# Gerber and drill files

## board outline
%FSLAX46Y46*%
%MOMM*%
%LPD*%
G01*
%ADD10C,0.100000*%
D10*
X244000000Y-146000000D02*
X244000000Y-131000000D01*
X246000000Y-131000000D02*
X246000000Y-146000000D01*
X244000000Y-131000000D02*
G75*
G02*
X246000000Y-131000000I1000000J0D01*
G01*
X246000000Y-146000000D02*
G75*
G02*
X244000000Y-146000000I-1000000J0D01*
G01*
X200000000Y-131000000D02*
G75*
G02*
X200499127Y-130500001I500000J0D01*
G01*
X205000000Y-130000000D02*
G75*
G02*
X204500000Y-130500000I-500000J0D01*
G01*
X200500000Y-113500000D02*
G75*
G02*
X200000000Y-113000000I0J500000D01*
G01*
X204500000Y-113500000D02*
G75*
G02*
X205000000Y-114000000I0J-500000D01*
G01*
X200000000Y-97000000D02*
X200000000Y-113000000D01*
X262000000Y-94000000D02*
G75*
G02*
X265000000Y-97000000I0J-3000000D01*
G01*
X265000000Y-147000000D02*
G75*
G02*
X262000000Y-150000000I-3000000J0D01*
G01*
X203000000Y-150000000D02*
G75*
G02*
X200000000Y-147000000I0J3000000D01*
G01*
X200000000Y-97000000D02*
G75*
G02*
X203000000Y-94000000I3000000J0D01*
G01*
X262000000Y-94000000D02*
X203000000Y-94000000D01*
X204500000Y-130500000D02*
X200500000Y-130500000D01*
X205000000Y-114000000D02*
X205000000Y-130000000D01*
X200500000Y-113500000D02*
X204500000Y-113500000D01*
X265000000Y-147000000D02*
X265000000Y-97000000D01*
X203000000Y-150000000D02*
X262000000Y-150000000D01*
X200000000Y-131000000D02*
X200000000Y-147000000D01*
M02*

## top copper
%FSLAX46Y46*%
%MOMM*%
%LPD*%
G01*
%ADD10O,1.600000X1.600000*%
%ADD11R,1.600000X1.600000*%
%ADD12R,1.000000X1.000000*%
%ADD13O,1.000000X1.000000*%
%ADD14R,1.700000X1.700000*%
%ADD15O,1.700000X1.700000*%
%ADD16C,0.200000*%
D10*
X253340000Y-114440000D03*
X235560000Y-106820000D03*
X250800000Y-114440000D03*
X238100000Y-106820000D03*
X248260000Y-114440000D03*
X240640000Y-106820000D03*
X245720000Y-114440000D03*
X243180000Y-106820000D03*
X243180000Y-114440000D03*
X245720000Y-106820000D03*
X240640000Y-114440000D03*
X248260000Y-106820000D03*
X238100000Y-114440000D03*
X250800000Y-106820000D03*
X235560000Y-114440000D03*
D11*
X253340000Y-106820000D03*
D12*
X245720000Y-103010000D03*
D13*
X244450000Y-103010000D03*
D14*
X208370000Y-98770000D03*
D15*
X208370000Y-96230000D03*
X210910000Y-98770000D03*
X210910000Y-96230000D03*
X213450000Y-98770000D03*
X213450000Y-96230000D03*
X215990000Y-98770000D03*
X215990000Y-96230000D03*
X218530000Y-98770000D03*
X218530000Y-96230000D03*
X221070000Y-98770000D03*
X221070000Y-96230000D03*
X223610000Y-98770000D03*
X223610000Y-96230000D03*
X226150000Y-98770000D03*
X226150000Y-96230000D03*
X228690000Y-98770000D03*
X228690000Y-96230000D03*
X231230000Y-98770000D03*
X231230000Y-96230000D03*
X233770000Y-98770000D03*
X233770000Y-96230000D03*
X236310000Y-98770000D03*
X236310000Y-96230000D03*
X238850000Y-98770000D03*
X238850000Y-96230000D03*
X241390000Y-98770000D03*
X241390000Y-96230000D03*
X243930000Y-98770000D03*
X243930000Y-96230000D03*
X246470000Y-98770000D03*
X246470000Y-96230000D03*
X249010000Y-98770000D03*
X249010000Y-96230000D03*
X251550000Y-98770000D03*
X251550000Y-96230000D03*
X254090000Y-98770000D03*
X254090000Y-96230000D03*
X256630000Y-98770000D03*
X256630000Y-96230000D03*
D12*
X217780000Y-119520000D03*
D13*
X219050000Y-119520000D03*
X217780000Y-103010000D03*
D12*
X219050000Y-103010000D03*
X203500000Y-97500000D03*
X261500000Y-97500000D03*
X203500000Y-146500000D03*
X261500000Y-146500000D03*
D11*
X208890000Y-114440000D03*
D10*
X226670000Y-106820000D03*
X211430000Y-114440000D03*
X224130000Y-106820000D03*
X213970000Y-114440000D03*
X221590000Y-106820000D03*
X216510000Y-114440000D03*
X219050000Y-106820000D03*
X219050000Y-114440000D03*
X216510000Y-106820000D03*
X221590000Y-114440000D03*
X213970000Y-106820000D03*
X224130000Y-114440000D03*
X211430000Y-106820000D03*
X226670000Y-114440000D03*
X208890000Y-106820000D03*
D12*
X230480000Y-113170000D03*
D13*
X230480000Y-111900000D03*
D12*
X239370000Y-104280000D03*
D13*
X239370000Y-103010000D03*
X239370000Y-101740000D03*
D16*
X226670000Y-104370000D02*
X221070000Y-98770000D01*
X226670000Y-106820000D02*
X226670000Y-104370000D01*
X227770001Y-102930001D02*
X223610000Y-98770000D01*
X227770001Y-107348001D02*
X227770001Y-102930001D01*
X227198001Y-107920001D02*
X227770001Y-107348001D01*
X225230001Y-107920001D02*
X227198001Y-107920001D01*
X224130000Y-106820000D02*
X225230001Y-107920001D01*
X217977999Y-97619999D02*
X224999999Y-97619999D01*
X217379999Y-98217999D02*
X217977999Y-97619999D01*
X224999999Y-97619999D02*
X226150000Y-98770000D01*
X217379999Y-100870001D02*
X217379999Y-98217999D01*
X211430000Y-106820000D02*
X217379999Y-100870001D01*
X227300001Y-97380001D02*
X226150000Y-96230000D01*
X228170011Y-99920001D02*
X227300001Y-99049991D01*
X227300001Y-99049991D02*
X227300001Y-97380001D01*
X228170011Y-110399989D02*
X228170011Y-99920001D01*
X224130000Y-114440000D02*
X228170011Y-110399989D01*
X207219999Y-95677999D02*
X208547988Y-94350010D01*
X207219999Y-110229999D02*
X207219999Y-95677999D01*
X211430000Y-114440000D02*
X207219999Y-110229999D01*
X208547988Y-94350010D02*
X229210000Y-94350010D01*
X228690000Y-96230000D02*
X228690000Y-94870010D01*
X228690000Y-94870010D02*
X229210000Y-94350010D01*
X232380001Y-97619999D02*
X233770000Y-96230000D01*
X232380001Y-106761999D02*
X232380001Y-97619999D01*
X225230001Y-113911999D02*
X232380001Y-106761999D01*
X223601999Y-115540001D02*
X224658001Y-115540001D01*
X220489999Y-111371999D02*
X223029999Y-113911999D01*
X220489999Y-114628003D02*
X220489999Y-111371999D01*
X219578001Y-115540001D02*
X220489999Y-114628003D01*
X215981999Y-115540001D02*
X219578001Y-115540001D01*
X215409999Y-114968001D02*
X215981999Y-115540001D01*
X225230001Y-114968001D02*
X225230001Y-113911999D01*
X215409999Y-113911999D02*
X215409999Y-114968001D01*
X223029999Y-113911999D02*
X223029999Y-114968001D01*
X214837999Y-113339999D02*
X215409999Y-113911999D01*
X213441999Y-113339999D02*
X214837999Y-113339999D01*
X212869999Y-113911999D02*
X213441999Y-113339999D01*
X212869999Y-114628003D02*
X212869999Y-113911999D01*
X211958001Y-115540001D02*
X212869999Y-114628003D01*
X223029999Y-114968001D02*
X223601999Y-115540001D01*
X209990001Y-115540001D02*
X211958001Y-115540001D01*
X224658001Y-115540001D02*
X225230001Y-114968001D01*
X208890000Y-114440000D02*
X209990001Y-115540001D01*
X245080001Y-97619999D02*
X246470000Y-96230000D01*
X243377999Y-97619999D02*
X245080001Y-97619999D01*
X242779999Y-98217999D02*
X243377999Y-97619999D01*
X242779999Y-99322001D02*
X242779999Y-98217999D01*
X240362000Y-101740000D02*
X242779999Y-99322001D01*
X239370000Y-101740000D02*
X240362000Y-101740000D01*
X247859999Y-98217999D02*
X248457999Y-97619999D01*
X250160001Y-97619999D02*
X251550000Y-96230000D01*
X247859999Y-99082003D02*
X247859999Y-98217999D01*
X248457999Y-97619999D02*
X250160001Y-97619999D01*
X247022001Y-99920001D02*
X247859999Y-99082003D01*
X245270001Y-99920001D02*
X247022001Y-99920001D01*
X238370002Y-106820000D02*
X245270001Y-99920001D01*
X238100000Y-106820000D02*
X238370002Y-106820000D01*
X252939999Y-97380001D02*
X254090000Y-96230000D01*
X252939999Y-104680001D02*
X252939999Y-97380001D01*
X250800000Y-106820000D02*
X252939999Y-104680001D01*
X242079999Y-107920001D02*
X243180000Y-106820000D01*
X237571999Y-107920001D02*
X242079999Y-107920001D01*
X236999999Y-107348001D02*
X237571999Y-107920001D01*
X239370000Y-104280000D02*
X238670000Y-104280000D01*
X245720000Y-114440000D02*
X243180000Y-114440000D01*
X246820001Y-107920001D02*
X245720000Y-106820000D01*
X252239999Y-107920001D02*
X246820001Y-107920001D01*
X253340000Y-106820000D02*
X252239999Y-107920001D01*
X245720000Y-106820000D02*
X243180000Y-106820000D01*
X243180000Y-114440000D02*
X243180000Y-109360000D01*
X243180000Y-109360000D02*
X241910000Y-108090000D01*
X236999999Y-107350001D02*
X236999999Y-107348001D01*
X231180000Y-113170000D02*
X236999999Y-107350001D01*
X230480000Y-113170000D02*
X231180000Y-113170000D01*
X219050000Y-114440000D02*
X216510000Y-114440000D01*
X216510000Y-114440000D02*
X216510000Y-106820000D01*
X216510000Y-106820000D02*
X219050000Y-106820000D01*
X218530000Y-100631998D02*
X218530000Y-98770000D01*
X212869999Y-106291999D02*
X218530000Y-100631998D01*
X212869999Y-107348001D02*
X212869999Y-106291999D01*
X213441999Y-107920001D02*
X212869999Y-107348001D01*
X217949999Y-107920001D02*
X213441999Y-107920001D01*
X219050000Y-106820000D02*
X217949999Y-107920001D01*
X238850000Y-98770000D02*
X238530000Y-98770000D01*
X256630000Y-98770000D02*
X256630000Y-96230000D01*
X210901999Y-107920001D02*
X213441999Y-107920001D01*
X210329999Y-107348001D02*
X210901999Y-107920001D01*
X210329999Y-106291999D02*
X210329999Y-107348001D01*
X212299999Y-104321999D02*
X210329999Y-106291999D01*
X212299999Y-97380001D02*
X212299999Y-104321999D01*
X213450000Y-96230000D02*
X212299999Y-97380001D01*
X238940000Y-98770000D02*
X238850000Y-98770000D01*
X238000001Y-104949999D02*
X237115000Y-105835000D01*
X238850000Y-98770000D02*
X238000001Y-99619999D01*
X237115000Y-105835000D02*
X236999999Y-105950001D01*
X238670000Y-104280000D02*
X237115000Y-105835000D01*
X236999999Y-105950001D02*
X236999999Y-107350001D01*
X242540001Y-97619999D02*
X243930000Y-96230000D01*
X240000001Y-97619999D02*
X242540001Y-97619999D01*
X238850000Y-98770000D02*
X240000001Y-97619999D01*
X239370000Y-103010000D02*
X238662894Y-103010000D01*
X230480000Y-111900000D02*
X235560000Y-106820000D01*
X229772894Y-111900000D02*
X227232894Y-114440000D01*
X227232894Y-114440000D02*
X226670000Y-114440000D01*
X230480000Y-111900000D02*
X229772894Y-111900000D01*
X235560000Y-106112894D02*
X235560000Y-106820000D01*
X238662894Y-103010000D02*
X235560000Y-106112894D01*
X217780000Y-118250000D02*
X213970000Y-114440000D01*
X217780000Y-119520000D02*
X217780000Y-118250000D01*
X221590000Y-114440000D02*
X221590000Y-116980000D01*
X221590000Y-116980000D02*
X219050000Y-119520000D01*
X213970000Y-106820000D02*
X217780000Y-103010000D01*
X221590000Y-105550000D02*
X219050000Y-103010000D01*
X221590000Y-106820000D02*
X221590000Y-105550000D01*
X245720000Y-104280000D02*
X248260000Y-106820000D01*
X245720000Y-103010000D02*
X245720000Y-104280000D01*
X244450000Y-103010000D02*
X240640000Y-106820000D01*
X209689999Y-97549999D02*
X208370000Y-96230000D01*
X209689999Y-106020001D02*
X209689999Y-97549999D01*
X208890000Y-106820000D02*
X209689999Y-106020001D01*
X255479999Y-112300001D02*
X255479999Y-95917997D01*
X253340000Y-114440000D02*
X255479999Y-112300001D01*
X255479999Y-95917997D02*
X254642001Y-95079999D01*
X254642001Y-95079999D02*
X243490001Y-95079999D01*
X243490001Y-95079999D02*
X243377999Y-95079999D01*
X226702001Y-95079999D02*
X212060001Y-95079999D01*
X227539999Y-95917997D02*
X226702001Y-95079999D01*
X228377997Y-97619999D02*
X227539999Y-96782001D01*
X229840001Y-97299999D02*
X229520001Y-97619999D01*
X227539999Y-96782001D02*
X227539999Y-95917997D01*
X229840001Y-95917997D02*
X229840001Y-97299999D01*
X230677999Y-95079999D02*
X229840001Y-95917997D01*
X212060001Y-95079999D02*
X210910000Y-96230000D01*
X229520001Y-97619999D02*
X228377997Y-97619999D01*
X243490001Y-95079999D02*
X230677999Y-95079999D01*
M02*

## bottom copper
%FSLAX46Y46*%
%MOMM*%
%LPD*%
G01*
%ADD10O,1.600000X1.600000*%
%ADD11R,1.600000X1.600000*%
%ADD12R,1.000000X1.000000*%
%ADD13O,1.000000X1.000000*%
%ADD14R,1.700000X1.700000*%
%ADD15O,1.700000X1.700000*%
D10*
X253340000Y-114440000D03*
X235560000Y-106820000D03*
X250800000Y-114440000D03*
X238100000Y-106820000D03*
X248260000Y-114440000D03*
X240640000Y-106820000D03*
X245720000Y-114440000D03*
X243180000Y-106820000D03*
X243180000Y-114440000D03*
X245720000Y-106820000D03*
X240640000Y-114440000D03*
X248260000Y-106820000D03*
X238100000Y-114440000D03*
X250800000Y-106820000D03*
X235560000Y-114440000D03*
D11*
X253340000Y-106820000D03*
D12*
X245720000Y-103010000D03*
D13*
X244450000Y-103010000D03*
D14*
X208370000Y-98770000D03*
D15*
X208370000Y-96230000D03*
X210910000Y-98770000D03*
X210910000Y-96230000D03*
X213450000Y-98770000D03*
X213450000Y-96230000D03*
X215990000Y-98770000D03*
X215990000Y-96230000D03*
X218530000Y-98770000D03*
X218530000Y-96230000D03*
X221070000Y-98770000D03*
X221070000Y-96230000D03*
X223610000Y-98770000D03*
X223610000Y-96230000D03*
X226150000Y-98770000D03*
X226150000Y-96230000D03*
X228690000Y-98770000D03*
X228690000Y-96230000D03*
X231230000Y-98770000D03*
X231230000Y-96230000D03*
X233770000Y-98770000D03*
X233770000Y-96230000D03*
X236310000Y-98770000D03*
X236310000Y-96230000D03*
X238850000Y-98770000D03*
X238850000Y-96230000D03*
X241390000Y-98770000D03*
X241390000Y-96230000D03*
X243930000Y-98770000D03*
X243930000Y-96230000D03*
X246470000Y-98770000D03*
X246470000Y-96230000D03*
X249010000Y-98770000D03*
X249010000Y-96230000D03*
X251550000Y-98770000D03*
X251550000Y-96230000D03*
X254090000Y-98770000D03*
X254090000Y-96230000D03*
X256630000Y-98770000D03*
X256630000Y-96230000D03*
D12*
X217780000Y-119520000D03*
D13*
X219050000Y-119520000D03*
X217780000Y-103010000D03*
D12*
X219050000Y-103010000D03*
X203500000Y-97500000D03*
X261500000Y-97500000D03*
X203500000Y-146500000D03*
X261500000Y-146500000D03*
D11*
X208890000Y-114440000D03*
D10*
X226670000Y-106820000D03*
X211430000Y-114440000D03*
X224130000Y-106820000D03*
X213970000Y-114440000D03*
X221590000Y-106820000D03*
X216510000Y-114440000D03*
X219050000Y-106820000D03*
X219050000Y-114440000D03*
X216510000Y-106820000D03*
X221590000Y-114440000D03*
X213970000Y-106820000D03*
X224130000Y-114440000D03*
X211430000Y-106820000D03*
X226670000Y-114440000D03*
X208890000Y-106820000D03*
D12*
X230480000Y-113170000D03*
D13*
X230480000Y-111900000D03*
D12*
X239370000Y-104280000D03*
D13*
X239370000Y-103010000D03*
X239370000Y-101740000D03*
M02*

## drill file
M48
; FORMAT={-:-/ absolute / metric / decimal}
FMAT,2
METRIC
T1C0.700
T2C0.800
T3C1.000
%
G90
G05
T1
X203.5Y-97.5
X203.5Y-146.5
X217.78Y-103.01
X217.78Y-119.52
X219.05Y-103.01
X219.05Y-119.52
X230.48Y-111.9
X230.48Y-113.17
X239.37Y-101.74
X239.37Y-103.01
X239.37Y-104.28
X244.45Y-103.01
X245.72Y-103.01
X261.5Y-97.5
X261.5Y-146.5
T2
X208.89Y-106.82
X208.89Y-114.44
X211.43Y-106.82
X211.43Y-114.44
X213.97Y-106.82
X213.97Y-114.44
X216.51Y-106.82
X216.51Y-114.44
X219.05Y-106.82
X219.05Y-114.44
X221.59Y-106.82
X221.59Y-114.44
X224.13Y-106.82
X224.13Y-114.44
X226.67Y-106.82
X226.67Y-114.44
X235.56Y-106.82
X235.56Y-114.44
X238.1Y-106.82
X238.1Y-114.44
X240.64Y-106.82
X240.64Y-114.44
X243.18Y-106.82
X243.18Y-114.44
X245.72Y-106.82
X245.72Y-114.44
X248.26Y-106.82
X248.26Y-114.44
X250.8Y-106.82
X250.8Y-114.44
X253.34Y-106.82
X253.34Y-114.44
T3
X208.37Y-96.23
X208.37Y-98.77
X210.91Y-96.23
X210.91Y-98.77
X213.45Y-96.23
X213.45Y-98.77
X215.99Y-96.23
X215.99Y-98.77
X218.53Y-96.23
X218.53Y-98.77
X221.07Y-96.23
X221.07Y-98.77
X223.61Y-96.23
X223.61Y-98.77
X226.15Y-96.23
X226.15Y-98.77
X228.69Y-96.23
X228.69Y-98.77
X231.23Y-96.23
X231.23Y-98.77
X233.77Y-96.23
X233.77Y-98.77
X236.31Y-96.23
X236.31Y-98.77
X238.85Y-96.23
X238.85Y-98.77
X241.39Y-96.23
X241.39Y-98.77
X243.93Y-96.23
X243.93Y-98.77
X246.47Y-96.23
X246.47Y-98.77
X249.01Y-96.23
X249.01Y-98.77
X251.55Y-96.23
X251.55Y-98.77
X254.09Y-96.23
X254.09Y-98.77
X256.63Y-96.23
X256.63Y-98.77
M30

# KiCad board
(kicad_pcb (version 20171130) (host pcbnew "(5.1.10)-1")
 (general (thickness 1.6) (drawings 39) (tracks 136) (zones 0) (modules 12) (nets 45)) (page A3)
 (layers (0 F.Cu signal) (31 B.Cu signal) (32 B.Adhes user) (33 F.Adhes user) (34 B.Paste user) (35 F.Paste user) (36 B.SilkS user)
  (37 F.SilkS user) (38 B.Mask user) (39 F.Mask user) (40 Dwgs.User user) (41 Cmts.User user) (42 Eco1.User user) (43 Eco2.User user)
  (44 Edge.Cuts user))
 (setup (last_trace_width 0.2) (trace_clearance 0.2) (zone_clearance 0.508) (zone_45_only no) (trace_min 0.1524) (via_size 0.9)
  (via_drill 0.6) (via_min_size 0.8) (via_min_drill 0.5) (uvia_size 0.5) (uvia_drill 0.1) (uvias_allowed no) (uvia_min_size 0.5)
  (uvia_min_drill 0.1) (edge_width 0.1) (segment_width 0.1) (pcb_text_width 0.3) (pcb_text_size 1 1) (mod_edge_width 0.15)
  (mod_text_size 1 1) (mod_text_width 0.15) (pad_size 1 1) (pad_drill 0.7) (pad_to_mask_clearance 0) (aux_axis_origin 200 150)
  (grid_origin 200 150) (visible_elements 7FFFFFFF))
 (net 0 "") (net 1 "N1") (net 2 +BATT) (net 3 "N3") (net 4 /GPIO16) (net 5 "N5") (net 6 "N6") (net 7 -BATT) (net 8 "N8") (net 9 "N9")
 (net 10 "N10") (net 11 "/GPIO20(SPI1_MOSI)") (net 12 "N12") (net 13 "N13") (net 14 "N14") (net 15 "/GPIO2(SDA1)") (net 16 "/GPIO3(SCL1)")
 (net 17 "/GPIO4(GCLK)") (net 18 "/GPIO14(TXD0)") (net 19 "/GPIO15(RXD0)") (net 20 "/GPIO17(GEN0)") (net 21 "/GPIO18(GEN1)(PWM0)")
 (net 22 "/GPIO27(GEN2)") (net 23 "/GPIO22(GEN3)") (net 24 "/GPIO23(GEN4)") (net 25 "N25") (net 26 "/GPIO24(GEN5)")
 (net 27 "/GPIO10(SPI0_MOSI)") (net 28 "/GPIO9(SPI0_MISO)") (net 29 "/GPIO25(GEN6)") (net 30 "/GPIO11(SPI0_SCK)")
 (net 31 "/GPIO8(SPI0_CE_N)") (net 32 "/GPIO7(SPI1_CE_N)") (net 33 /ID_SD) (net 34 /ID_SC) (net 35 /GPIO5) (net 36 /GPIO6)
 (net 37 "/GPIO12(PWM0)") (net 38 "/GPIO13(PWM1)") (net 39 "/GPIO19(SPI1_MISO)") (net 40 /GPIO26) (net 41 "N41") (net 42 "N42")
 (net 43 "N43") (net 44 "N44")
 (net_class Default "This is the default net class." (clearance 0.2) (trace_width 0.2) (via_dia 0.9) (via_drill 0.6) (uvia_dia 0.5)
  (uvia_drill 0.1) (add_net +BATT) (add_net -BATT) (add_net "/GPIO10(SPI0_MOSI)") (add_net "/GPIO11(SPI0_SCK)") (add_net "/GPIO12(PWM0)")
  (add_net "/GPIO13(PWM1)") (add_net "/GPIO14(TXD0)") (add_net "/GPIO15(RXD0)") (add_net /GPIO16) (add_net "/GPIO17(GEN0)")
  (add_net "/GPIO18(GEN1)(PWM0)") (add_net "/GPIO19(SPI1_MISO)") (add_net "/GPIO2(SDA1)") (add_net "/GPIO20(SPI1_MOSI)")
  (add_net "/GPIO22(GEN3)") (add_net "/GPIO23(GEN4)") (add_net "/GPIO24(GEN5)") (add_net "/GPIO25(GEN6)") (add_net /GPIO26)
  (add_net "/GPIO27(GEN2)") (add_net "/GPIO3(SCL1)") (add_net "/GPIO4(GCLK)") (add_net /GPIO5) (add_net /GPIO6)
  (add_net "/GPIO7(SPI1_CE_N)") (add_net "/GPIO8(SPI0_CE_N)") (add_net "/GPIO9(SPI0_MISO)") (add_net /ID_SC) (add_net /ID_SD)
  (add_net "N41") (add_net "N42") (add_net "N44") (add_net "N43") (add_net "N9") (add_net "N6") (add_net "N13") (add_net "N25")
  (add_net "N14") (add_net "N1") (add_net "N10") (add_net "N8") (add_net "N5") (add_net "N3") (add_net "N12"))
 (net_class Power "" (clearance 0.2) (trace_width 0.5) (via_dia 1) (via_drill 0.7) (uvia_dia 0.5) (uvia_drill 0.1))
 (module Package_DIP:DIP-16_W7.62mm (layer F.Cu) (at 253.34 106.82 270)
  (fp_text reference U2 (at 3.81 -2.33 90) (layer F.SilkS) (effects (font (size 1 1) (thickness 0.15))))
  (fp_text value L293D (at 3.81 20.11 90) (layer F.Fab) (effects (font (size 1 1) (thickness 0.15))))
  (pad 16 thru_hole oval (at 7.62 0 270) (size 1.6 1.6) (drill 0.8) (layers *.Cu *.Mask) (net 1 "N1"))
  (pad 8 thru_hole oval (at 0 17.78 270) (size 1.6 1.6) (drill 0.8) (layers *.Cu *.Mask) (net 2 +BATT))
  (pad 15 thru_hole oval (at 7.62 2.54 270) (size 1.6 1.6) (drill 0.8) (layers *.Cu *.Mask) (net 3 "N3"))
  (pad 7 thru_hole oval (at 0 15.24 270) (size 1.6 1.6) (drill 0.8) (layers *.Cu *.Mask) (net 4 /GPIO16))
  (pad 14 thru_hole oval (at 7.62 5.08 270) (size 1.6 1.6) (drill 0.8) (layers *.Cu *.Mask) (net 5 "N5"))
  (pad 6 thru_hole oval (at 0 12.7 270) (size 1.6 1.6) (drill 0.8) (layers *.Cu *.Mask) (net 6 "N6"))
  (pad 13 thru_hole oval (at 7.62 7.62 270) (size 1.6 1.6) (drill 0.8) (layers *.Cu *.Mask) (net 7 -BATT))
  (pad 5 thru_hole oval (at 0 10.16 270) (size 1.6 1.6) (drill 0.8) (layers *.Cu *.Mask) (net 7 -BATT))
  (pad 12 thru_hole oval (at 7.62 10.16 270) (size 1.6 1.6) (drill 0.8) (layers *.Cu *.Mask) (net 7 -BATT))
  (pad 4 thru_hole oval (at 0 7.62 270) (size 1.6 1.6) (drill 0.8) (layers *.Cu *.Mask) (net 7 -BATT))
  (pad 11 thru_hole oval (at 7.62 12.7 270) (size 1.6 1.6) (drill 0.8) (layers *.Cu *.Mask) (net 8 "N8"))
  (pad 3 thru_hole oval (at 0 5.08 270) (size 1.6 1.6) (drill 0.8) (layers *.Cu *.Mask) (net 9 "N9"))
  (pad 10 thru_hole oval (at 7.62 15.24 270) (size 1.6 1.6) (drill 0.8) (layers *.Cu *.Mask) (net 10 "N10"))
  (pad 2 thru_hole oval (at 0 2.54 270) (size 1.6 1.6) (drill 0.8) (layers *.Cu *.Mask) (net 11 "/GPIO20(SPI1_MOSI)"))
  (pad 9 thru_hole oval (at 7.62 17.78 270) (size 1.6 1.6) (drill 0.8) (layers *.Cu *.Mask) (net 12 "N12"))
  (pad 1 thru_hole rect (at 0 0 270) (size 1.6 1.6) (drill 0.8) (layers *.Cu *.Mask) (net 7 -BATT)))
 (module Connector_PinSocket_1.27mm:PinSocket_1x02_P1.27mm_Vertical (layer F.Cu) (at 245.72 103.01 270)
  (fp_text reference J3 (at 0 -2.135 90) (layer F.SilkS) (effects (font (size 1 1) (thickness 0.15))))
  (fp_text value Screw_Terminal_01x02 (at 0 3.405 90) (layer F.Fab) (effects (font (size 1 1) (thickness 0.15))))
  (pad 1 thru_hole rect (at 0 0 270) (size 1 1) (drill 0.7) (layers *.Cu *.Mask) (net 9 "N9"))
  (pad 2 thru_hole oval (at 0 1.27 270) (size 1 1) (drill 0.7) (layers *.Cu *.Mask) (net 6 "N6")))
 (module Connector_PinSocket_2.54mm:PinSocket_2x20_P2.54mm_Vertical (layer B.Cu) (at 208.37 98.77 270)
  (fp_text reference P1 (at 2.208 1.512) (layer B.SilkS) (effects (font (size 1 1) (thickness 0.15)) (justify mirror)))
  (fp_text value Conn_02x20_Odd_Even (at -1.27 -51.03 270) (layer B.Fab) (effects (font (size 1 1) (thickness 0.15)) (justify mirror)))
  (pad 1 thru_hole rect (at 0 0 270) (size 1.7 1.7) (drill 1) (layers *.Cu *.Mask) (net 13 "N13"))
  (pad 2 thru_hole oval (at -2.54 0 270) (size 1.7 1.7) (drill 1) (layers *.Cu *.Mask) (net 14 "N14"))
  (pad 3 thru_hole oval (at 0 -2.54 270) (size 1.7 1.7) (drill 1) (layers *.Cu *.Mask) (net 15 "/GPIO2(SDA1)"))
  (pad 4 thru_hole oval (at -2.54 -2.54 270) (size 1.7 1.7) (drill 1) (layers *.Cu *.Mask) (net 1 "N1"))
  (pad 5 thru_hole oval (at 0 -5.08 270) (size 1.7 1.7) (drill 1) (layers *.Cu *.Mask) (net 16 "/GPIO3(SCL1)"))
  (pad 6 thru_hole oval (at -2.54 -5.08 270) (size 1.7 1.7) (drill 1) (layers *.Cu *.Mask) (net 7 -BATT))
  (pad 7 thru_hole oval (at 0 -7.62 270) (size 1.7 1.7) (drill 1) (layers *.Cu *.Mask) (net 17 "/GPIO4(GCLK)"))
  (pad 8 thru_hole oval (at -2.54 -7.62 270) (size 1.7 1.7) (drill 1) (layers *.Cu *.Mask) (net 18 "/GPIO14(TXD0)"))
  (pad 9 thru_hole oval (at 0 -10.16 270) (size 1.7 1.7) (drill 1) (layers *.Cu *.Mask) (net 7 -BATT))
  (pad 10 thru_hole oval (at -2.54 -10.16 270) (size 1.7 1.7) (drill 1) (layers *.Cu *.Mask) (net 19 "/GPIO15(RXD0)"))
  (pad 11 thru_hole oval (at 0 -12.7 270) (size 1.7 1.7) (drill 1) (layers *.Cu *.Mask) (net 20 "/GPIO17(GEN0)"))
  (pad 12 thru_hole oval (at -2.54 -12.7 270) (size 1.7 1.7) (drill 1) (layers *.Cu *.Mask) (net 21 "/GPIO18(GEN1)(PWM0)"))
  (pad 13 thru_hole oval (at 0 -15.24 270) (size 1.7 1.7) (drill 1) (layers *.Cu *.Mask) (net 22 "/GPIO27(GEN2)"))
  (pad 14 thru_hole oval (at -2.54 -15.24 270) (size 1.7 1.7) (drill 1) (layers *.Cu *.Mask) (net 7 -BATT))
  (pad 15 thru_hole oval (at 0 -17.78 270) (size 1.7 1.7) (drill 1) (layers *.Cu *.Mask) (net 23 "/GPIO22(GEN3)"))
  (pad 16 thru_hole oval (at -2.54 -17.78 270) (size 1.7 1.7) (drill 1) (layers *.Cu *.Mask) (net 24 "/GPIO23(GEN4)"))
  (pad 17 thru_hole oval (at 0 -20.32 270) (size 1.7 1.7) (drill 1) (layers *.Cu *.Mask) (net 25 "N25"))
  (pad 18 thru_hole oval (at -2.54 -20.32 270) (size 1.7 1.7) (drill 1) (layers *.Cu *.Mask) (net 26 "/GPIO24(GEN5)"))
  (pad 19 thru_hole oval (at 0 -22.86 270) (size 1.7 1.7) (drill 1) (layers *.Cu *.Mask) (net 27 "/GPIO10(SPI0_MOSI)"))
  (pad 20 thru_hole oval (at -2.54 -22.86 270) (size 1.7 1.7) (drill 1) (layers *.Cu *.Mask) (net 7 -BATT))
  (pad 21 thru_hole oval (at 0 -25.4 270) (size 1.7 1.7) (drill 1) (layers *.Cu *.Mask) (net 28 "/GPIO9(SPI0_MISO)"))
  (pad 22 thru_hole oval (at -2.54 -25.4 270) (size 1.7 1.7) (drill 1) (layers *.Cu *.Mask) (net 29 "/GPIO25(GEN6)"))
  (pad 23 thru_hole oval (at 0 -27.94 270) (size 1.7 1.7) (drill 1) (layers *.Cu *.Mask) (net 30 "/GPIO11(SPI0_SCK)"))
  (pad 24 thru_hole oval (at -2.54 -27.94 270) (size 1.7 1.7) (drill 1) (layers *.Cu *.Mask) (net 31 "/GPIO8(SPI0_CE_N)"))
  (pad 25 thru_hole oval (at 0 -30.48 270) (size 1.7 1.7) (drill 1) (layers *.Cu *.Mask) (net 7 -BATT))
  (pad 26 thru_hole oval (at -2.54 -30.48 270) (size 1.7 1.7) (drill 1) (layers *.Cu *.Mask) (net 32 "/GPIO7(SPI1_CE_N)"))
  (pad 27 thru_hole oval (at 0 -33.02 270) (size 1.7 1.7) (drill 1) (layers *.Cu *.Mask) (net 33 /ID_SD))
  (pad 28 thru_hole oval (at -2.54 -33.02 270) (size 1.7 1.7) (drill 1) (layers *.Cu *.Mask) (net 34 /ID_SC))
  (pad 29 thru_hole oval (at 0 -35.56 270) (size 1.7 1.7) (drill 1) (layers *.Cu *.Mask) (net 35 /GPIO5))
  (pad 30 thru_hole oval (at -2.54 -35.56 270) (size 1.7 1.7) (drill 1) (layers *.Cu *.Mask) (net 7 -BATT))
  (pad 31 thru_hole oval (at 0 -38.1 270) (size 1.7 1.7) (drill 1) (layers *.Cu *.Mask) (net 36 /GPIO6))
  (pad 32 thru_hole oval (at -2.54 -38.1 270) (size 1.7 1.7) (drill 1) (layers *.Cu *.Mask) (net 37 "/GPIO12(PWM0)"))
  (pad 33 thru_hole oval (at 0 -40.64 270) (size 1.7 1.7) (drill 1) (layers *.Cu *.Mask) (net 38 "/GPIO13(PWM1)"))
  (pad 34 thru_hole oval (at -2.54 -40.64 270) (size 1.7 1.7) (drill 1) (layers *.Cu *.Mask) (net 7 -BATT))
  (pad 35 thru_hole oval (at 0 -43.18 270) (size 1.7 1.7) (drill 1) (layers *.Cu *.Mask) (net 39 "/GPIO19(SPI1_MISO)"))
  (pad 36 thru_hole oval (at -2.54 -43.18 270) (size 1.7 1.7) (drill 1) (layers *.Cu *.Mask) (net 4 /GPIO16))
  (pad 37 thru_hole oval (at 0 -45.72 270) (size 1.7 1.7) (drill 1) (layers *.Cu *.Mask) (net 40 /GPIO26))
  (pad 38 thru_hole oval (at -2.54 -45.72 270) (size 1.7 1.7) (drill 1) (layers *.Cu *.Mask) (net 11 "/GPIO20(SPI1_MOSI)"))
  (pad 39 thru_hole oval (at 0 -48.26 270) (size 1.7 1.7) (drill 1) (layers *.Cu *.Mask) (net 7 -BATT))
  (pad 40 thru_hole oval (at -2.54 -48.26 270) (size 1.7 1.7) (drill 1) (layers *.Cu *.Mask) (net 7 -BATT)))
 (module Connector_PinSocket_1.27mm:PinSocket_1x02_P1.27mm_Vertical (layer F.Cu) (at 217.78 119.52 90)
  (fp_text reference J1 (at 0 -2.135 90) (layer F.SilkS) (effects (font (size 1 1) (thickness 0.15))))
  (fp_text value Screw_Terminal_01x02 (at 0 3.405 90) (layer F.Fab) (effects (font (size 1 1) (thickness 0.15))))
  (pad 1 thru_hole rect (at 0 0 90) (size 1 1) (drill 0.7) (layers *.Cu *.Mask) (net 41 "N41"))
  (pad 2 thru_hole oval (at 0 1.27 90) (size 1 1) (drill 0.7) (layers *.Cu *.Mask) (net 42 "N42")))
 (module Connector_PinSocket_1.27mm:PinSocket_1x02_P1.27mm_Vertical (layer F.Cu) (at 219.05 103.01 270)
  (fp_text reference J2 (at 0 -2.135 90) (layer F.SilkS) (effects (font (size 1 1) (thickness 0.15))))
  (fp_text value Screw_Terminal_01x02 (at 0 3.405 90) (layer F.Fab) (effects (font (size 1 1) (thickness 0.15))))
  (pad 2 thru_hole oval (at 0 1.27 270) (size 1 1) (drill 0.7) (layers *.Cu *.Mask) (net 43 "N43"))
  (pad 1 thru_hole rect (at 0 0 270) (size 1 1) (drill 0.7) (layers *.Cu *.Mask) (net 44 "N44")))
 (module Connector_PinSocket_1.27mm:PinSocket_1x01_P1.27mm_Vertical (layer F.Cu) (at 203.5 97.5 180)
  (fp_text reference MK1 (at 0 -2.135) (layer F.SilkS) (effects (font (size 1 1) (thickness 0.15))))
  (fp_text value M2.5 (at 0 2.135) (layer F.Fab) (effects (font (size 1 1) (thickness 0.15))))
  (pad 1 thru_hole rect (at 0 0 180) (size 1 1) (drill 0.7) (layers *.Cu *.Mask)))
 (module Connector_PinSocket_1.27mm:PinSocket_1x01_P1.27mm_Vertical (layer F.Cu) (at 261.5 97.5 180)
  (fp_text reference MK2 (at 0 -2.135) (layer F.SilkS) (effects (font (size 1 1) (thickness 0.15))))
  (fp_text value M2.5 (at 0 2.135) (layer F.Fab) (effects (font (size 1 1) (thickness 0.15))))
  (pad 1 thru_hole rect (at 0 0 180) (size 1 1) (drill 0.7) (layers *.Cu *.Mask)))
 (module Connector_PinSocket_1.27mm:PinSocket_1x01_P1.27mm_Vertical (layer F.Cu) (at 203.5 146.5)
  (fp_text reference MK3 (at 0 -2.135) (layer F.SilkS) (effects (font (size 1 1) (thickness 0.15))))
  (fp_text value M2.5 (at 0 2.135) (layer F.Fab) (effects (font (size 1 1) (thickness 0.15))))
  (pad 1 thru_hole rect (at 0 0) (size 1 1) (drill 0.7) (layers *.Cu *.Mask)))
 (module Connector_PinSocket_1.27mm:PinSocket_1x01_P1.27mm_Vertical (layer F.Cu) (at 261.5 146.5)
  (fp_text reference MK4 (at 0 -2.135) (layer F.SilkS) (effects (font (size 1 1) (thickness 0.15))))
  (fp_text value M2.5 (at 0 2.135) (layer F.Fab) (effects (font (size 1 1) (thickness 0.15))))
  (pad 1 thru_hole rect (at 0 0) (size 1 1) (drill 0.7) (layers *.Cu *.Mask)))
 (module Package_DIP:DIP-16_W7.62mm (layer F.Cu) (at 208.89 114.44 90)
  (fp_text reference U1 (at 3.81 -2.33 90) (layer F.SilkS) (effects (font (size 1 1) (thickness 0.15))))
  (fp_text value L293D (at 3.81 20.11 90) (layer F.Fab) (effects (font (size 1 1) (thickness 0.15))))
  (pad 1 thru_hole rect (at 0 0 90) (size 1.6 1.6) (drill 0.8) (layers *.Cu *.Mask) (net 29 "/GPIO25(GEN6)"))
  (pad 9 thru_hole oval (at 7.62 17.78 90) (size 1.6 1.6) (drill 0.8) (layers *.Cu *.Mask) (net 20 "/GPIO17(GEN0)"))
  (pad 2 thru_hole oval (at 0 2.54 90) (size 1.6 1.6) (drill 0.8) (layers *.Cu *.Mask) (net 26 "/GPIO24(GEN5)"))
  (pad 10 thru_hole oval (at 7.62 15.24 90) (size 1.6 1.6) (drill 0.8) (layers *.Cu *.Mask) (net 22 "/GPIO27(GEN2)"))
  (pad 3 thru_hole oval (at 0 5.08 90) (size 1.6 1.6) (drill 0.8) (layers *.Cu *.Mask) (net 41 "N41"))
  (pad 11 thru_hole oval (at 7.62 12.7 90) (size 1.6 1.6) (drill 0.8) (layers *.Cu *.Mask) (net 44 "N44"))
  (pad 4 thru_hole oval (at 0 7.62 90) (size 1.6 1.6) (drill 0.8) (layers *.Cu *.Mask) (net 7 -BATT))
  (pad 12 thru_hole oval (at 7.62 10.16 90) (size 1.6 1.6) (drill 0.8) (layers *.Cu *.Mask) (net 7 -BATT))
  (pad 5 thru_hole oval (at 0 10.16 90) (size 1.6 1.6) (drill 0.8) (layers *.Cu *.Mask) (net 7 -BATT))
  (pad 13 thru_hole oval (at 7.62 7.62 90) (size 1.6 1.6) (drill 0.8) (layers *.Cu *.Mask) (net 7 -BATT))
  (pad 6 thru_hole oval (at 0 12.7 90) (size 1.6 1.6) (drill 0.8) (layers *.Cu *.Mask) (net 42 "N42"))
  (pad 14 thru_hole oval (at 7.62 5.08 90) (size 1.6 1.6) (drill 0.8) (layers *.Cu *.Mask) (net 43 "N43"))
  (pad 7 thru_hole oval (at 0 15.24 90) (size 1.6 1.6) (drill 0.8) (layers *.Cu *.Mask) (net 24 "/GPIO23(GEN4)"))
  (pad 15 thru_hole oval (at 7.62 2.54 90) (size 1.6 1.6) (drill 0.8) (layers *.Cu *.Mask) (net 23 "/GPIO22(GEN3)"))
  (pad 8 thru_hole oval (at 0 17.78 90) (size 1.6 1.6) (drill 0.8) (layers *.Cu *.Mask) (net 2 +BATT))
  (pad 16 thru_hole oval (at 7.62 0 90) (size 1.6 1.6) (drill 0.8) (layers *.Cu *.Mask) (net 14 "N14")))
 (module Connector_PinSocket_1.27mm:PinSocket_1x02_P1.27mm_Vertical (layer F.Cu) (at 230.48 113.17 180)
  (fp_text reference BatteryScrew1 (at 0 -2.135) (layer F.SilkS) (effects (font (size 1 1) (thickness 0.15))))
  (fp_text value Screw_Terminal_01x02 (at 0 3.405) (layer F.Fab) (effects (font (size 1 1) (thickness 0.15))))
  (pad 1 thru_hole rect (at 0 0 180) (size 1 1) (drill 0.7) (layers *.Cu *.Mask) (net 7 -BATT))
  (pad 2 thru_hole oval (at 0 1.27 180) (size 1 1) (drill 0.7) (layers *.Cu *.Mask) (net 2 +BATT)))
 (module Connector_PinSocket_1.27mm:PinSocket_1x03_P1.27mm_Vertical (layer F.Cu) (at 239.37 104.28 180)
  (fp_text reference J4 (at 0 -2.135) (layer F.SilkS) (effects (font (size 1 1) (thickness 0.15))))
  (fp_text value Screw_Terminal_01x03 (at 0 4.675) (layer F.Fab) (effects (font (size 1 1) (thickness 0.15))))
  (pad 1 thru_hole rect (at 0 0 180) (size 1 1) (drill 0.7) (layers *.Cu *.Mask) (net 7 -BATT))
  (pad 2 thru_hole oval (at 0 1.27 180) (size 1 1) (drill 0.7) (layers *.Cu *.Mask) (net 2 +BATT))
  (pad 3 thru_hole oval (at 0 2.54 180) (size 1 1) (drill 0.7) (layers *.Cu *.Mask) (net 37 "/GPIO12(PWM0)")))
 (gr_line (start 244 146) (end 244 131) (layer Edge.Cuts) (width 0.1))
 (gr_line (start 246 131) (end 246 146) (layer Edge.Cuts) (width 0.1))
 (gr_arc (start 245 131) (end 244 131) (angle 180) (layer Edge.Cuts) (width 0.1))
 (gr_arc (start 245 146) (end 246 146) (angle 180) (layer Edge.Cuts) (width 0.1))
 (gr_arc (start 200.5 131) (end 200 131) (angle 89.9) (layer Edge.Cuts) (width 0.1))
 (gr_arc (start 204.5 130) (end 205 130) (angle 90) (layer Edge.Cuts) (width 0.1))
 (gr_arc (start 200.5 113) (end 200.5 113.5) (angle 90) (layer Edge.Cuts) (width 0.1))
 (gr_arc (start 204.5 114) (end 204.5 113.5) (angle 90) (layer Edge.Cuts) (width 0.1))
 (gr_line (start 200 97) (end 200 113) (layer Edge.Cuts) (width 0.1))
 (gr_arc (start 262 97) (end 262 94) (angle 90) (layer Edge.Cuts) (width 0.1))
 (gr_arc (start 262 147) (end 265 147) (angle 90) (layer Edge.Cuts) (width 0.1))
 (gr_arc (start 203 147) (end 203 150) (angle 90) (layer Edge.Cuts) (width 0.1))
 (gr_arc (start 203 97) (end 200 97) (angle 90) (layer Edge.Cuts) (width 0.1))
 (gr_line (start 262 94) (end 203 94) (layer Edge.Cuts) (width 0.1))
 (gr_line (start 204.5 130.5) (end 200.5 130.5) (layer Edge.Cuts) (width 0.1))
 (gr_line (start 205 114) (end 205 130) (layer Edge.Cuts) (width 0.1))
 (gr_line (start 200.5 113.5) (end 204.5 113.5) (layer Edge.Cuts) (width 0.1))
 (gr_line (start 265 147) (end 265 97) (layer Edge.Cuts) (width 0.1))
 (gr_line (start 203 150) (end 262 150) (layer Edge.Cuts) (width 0.1))
 (gr_line (start 200 131) (end 200 147) (layer Edge.Cuts) (width 0.1))
 (segment (start 226.67 104.37) (end 221.07 98.77) (width 0.2) (layer F.Cu) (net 20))
 (segment (start 226.67 106.82) (end 226.67 104.37) (width 0.2) (layer F.Cu) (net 20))
 (segment (start 227.770001 102.930001) (end 223.61 98.77) (width 0.2) (layer F.Cu) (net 22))
 (segment (start 227.770001 107.348001) (end 227.770001 102.930001) (width 0.2) (layer F.Cu) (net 22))
 (segment (start 227.198001 107.920001) (end 227.770001 107.348001) (width 0.2) (layer F.Cu) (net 22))
 (segment (start 225.230001 107.920001) (end 227.198001 107.920001) (width 0.2) (layer F.Cu) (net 22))
 (segment (start 224.13 106.82) (end 225.230001 107.920001) (width 0.2) (layer F.Cu) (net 22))
 (segment (start 217.977999 97.619999) (end 224.999999 97.619999) (width 0.2) (layer F.Cu) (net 23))
 (segment (start 217.379999 98.217999) (end 217.977999 97.619999) (width 0.2) (layer F.Cu) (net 23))
 (segment (start 224.999999 97.619999) (end 226.15 98.77) (width 0.2) (layer F.Cu) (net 23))
 (segment (start 217.379999 100.870001) (end 217.379999 98.217999) (width 0.2) (layer F.Cu) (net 23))
 (segment (start 211.43 106.82) (end 217.379999 100.870001) (width 0.2) (layer F.Cu) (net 23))
 (segment (start 227.300001 97.380001) (end 226.15 96.23) (width 0.2) (layer F.Cu) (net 24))
 (segment (start 228.170011 99.920001) (end 227.300001 99.049991) (width 0.2) (layer F.Cu) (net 24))
 (segment (start 227.300001 99.049991) (end 227.300001 97.380001) (width 0.2) (layer F.Cu) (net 24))
 (segment (start 228.170011 110.399989) (end 228.170011 99.920001) (width 0.2) (layer F.Cu) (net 24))
 (segment (start 224.13 114.44) (end 228.170011 110.399989) (width 0.2) (layer F.Cu) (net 24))
 (segment (start 207.219999 95.677999) (end 208.547988 94.35001) (width 0.2) (layer F.Cu) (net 26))
 (segment (start 207.219999 110.229999) (end 207.219999 95.677999) (width 0.2) (layer F.Cu) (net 26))
 (segment (start 211.43 114.44) (end 207.219999 110.229999) (width 0.2) (layer F.Cu) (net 26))
 (segment (start 208.547988 94.35001) (end 229.21 94.35001) (width 0.2) (layer F.Cu) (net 26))
 (segment (start 228.69 96.23) (end 228.69 94.87001) (width 0.2) (layer F.Cu) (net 26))
 (segment (start 228.69 94.87001) (end 229.21 94.35001) (width 0.2) (layer F.Cu) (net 26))
 (segment (start 232.380001 97.619999) (end 233.77 96.23) (width 0.2) (layer F.Cu) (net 29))
 (segment (start 232.380001 106.761999) (end 232.380001 97.619999) (width 0.2) (layer F.Cu) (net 29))
 (segment (start 225.230001 113.911999) (end 232.380001 106.761999) (width 0.2) (layer F.Cu) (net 29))
 (segment (start 223.601999 115.540001) (end 224.658001 115.540001) (width 0.2) (layer F.Cu) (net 29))
 (segment (start 220.489999 111.371999) (end 223.029999 113.911999) (width 0.2) (layer F.Cu) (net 29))
 (segment (start 220.489999 114.628003) (end 220.489999 111.371999) (width 0.2) (layer F.Cu) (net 29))
 (segment (start 219.578001 115.540001) (end 220.489999 114.628003) (width 0.2) (layer F.Cu) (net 29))
 (segment (start 215.981999 115.540001) (end 219.578001 115.540001) (width 0.2) (layer F.Cu) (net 29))
 (segment (start 215.409999 114.968001) (end 215.981999 115.540001) (width 0.2) (layer F.Cu) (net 29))
 (segment (start 225.230001 114.968001) (end 225.230001 113.911999) (width 0.2) (layer F.Cu) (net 29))
 (segment (start 215.409999 113.911999) (end 215.409999 114.968001) (width 0.2) (layer F.Cu) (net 29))
 (segment (start 223.029999 113.911999) (end 223.029999 114.968001) (width 0.2) (layer F.Cu) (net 29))
 (segment (start 214.837999 113.339999) (end 215.409999 113.911999) (width 0.2) (layer F.Cu) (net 29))
 (segment (start 213.441999 113.339999) (end 214.837999 113.339999) (width 0.2) (layer F.Cu) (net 29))
 (segment (start 212.869999 113.911999) (end 213.441999 113.339999) (width 0.2) (layer F.Cu) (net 29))
 (segment (start 212.869999 114.628003) (end 212.869999 113.911999) (width 0.2) (layer F.Cu) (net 29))
 (segment (start 211.958001 115.540001) (end 212.869999 114.628003) (width 0.2) (layer F.Cu) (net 29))
 (segment (start 223.029999 114.968001) (end 223.601999 115.540001) (width 0.2) (layer F.Cu) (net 29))
 (segment (start 209.990001 115.540001) (end 211.958001 115.540001) (width 0.2) (layer F.Cu) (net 29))
 (segment (start 224.658001 115.540001) (end 225.230001 114.968001) (width 0.2) (layer F.Cu) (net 29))
 (segment (start 208.89 114.44) (end 209.990001 115.540001) (width 0.2) (layer F.Cu) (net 29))
 (segment (start 245.080001 97.619999) (end 246.47 96.23) (width 0.2) (layer F.Cu) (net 37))
 (segment (start 243.377999 97.619999) (end 245.080001 97.619999) (width 0.2) (layer F.Cu) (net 37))
 (segment (start 242.779999 98.217999) (end 243.377999 97.619999) (width 0.2) (layer F.Cu) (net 37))
 (segment (start 242.779999 99.322001) (end 242.779999 98.217999) (width 0.2) (layer F.Cu) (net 37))
 (segment (start 240.362 101.74) (end 242.779999 99.322001) (width 0.2) (layer F.Cu) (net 37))
 (segment (start 239.37 101.74) (end 240.362 101.74) (width 0.2) (layer F.Cu) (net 37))
 (segment (start 247.859999 98.217999) (end 248.457999 97.619999) (width 0.2) (layer F.Cu) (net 4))
 (segment (start 250.160001 97.619999) (end 251.55 96.23) (width 0.2) (layer F.Cu) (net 4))
 (segment (start 247.859999 99.082003) (end 247.859999 98.217999) (width 0.2) (layer F.Cu) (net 4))
 (segment (start 248.457999 97.619999) (end 250.160001 97.619999) (width 0.2) (layer F.Cu) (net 4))
 (segment (start 247.022001 99.920001) (end 247.859999 99.082003) (width 0.2) (layer F.Cu) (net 4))
 (segment (start 245.270001 99.920001) (end 247.022001 99.920001) (width 0.2) (layer F.Cu) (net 4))
 (segment (start 238.370002 106.82) (end 245.270001 99.920001) (width 0.2) (layer F.Cu) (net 4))
 (segment (start 238.1 106.82) (end 238.370002 106.82) (width 0.2) (layer F.Cu) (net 4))
 (segment (start 252.939999 97.380001) (end 254.09 96.23) (width 0.2) (layer F.Cu) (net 11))
 (segment (start 252.939999 104.680001) (end 252.939999 97.380001) (width 0.2) (layer F.Cu) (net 11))
 (segment (start 250.8 106.82) (end 252.939999 104.680001) (width 0.2) (layer F.Cu) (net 11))
 (segment (start 242.079999 107.920001) (end 243.18 106.82) (width 0.2) (layer F.Cu) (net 7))
 (segment (start 237.571999 107.920001) (end 242.079999 107.920001) (width 0.2) (layer F.Cu) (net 7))
 (segment (start 236.999999 107.348001) (end 237.571999 107.920001) (width 0.2) (layer F.Cu) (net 7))
 (segment (start 239.37 104.28) (end 238.67 104.28) (width 0.2) (layer F.Cu) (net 7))
 (segment (start 245.72 114.44) (end 243.18 114.44) (width 0.2) (layer F.Cu) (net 7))
 (segment (start 246.820001 107.920001) (end 245.72 106.82) (width 0.2) (layer F.Cu) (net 7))
 (segment (start 252.239999 107.920001) (end 246.820001 107.920001) (width 0.2) (layer F.Cu) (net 7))
 (segment (start 253.34 106.82) (end 252.239999 107.920001) (width 0.2) (layer F.Cu) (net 7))
 (segment (start 245.72 106.82) (end 243.18 106.82) (width 0.2) (layer F.Cu) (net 7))
 (segment (start 243.18 114.44) (end 243.18 109.36) (width 0.2) (layer F.Cu) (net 7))
 (segment (start 243.18 109.36) (end 241.91 108.09) (width 0.2) (layer F.Cu) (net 7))
 (segment (start 236.999999 107.350001) (end 236.999999 107.348001) (width 0.2) (layer F.Cu) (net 7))
 (segment (start 231.18 113.17) (end 236.999999 107.350001) (width 0.2) (layer F.Cu) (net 7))
 (segment (start 230.48 113.17) (end 231.18 113.17) (width 0.2) (layer F.Cu) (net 7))
 (segment (start 219.05 114.44) (end 216.51 114.44) (width 0.2) (layer F.Cu) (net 7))
 (segment (start 216.51 114.44) (end 216.51 106.82) (width 0.2) (layer F.Cu) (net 7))
 (segment (start 216.51 106.82) (end 219.05 106.82) (width 0.2) (layer F.Cu) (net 7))
 (segment (start 218.53 100.631998) (end 218.53 98.77) (width 0.2) (layer F.Cu) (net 7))
 (segment (start 212.869999 106.291999) (end 218.53 100.631998) (width 0.2) (layer F.Cu) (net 7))
 (segment (start 212.869999 107.348001) (end 212.869999 106.291999) (width 0.2) (layer F.Cu) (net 7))
 (segment (start 213.441999 107.920001) (end 212.869999 107.348001) (width 0.2) (layer F.Cu) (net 7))
 (segment (start 217.949999 107.920001) (end 213.441999 107.920001) (width 0.2) (layer F.Cu) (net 7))
 (segment (start 219.05 106.82) (end 217.949999 107.920001) (width 0.2) (layer F.Cu) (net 7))
 (segment (start 238.85 98.77) (end 238.53 98.77) (width 0.2) (layer F.Cu) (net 7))
 (segment (start 256.63 98.77) (end 256.63 96.23) (width 0.2) (layer F.Cu) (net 7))
 (segment (start 210.901999 107.920001) (end 213.441999 107.920001) (width 0.2) (layer F.Cu) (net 7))
 (segment (start 210.329999 107.348001) (end 210.901999 107.920001) (width 0.2) (layer F.Cu) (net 7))
 (segment (start 210.329999 106.291999) (end 210.329999 107.348001) (width 0.2) (layer F.Cu) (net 7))
 (segment (start 212.299999 104.321999) (end 210.329999 106.291999) (width 0.2) (layer F.Cu) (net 7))
 (segment (start 212.299999 97.380001) (end 212.299999 104.321999) (width 0.2) (layer F.Cu) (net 7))
 (segment (start 213.45 96.23) (end 212.299999 97.380001) (width 0.2) (layer F.Cu) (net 7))
 (segment (start 238.94 98.77) (end 238.85 98.77) (width 0.2) (layer F.Cu) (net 7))
 (segment (start 238.000001 104.949999) (end 237.115 105.835) (width 0.2) (layer F.Cu) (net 7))
 (segment (start 238.85 98.77) (end 238.000001 99.619999) (width 0.2) (layer F.Cu) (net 7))
 (segment (start 237.115 105.835) (end 236.999999 105.950001) (width 0.2) (layer F.Cu) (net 7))
 (segment (start 238.67 104.28) (end 237.115 105.835) (width 0.2) (layer F.Cu) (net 7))
 (segment (start 236.999999 105.950001) (end 236.999999 107.350001) (width 0.2) (layer F.Cu) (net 7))
 (segment (start 242.540001 97.619999) (end 243.93 96.23) (width 0.2) (layer F.Cu) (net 7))
 (segment (start 240.000001 97.619999) (end 242.540001 97.619999) (width 0.2) (layer F.Cu) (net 7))
 (segment (start 238.85 98.77) (end 240.000001 97.619999) (width 0.2) (layer F.Cu) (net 7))
 (segment (start 239.37 103.01) (end 238.662894 103.01) (width 0.2) (layer F.Cu) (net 2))
 (segment (start 230.48 111.9) (end 235.56 106.82) (width 0.2) (layer F.Cu) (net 2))
 (segment (start 229.772894 111.9) (end 227.232894 114.44) (width 0.2) (layer F.Cu) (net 2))
 (segment (start 227.232894 114.44) (end 226.67 114.44) (width 0.2) (layer F.Cu) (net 2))
 (segment (start 230.48 111.9) (end 229.772894 111.9) (width 0.2) (layer F.Cu) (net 2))
 (segment (start 235.56 106.112894) (end 235.56 106.82) (width 0.2) (layer F.Cu) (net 2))
 (segment (start 238.662894 103.01) (end 235.56 106.112894) (width 0.2) (layer F.Cu) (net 2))
 (segment (start 217.78 118.25) (end 213.97 114.44) (width 0.2) (layer F.Cu) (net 41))
 (segment (start 217.78 119.52) (end 217.78 118.25) (width 0.2) (layer F.Cu) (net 41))
 (segment (start 221.59 114.44) (end 221.59 116.98) (width 0.2) (layer F.Cu) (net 42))
 (segment (start 221.59 116.98) (end 219.05 119.52) (width 0.2) (layer F.Cu) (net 42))
 (segment (start 213.97 106.82) (end 217.78 103.01) (width 0.2) (layer F.Cu) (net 43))
 (segment (start 221.59 105.55) (end 219.05 103.01) (width 0.2) (layer F.Cu) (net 44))
 (segment (start 221.59 106.82) (end 221.59 105.55) (width 0.2) (layer F.Cu) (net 44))
 (segment (start 245.72 104.28) (end 248.26 106.82) (width 0.2) (layer F.Cu) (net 9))
 (segment (start 245.72 103.01) (end 245.72 104.28) (width 0.2) (layer F.Cu) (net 9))
 (segment (start 244.45 103.01) (end 240.64 106.82) (width 0.2) (layer F.Cu) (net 6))
 (segment (start 209.689999 97.549999) (end 208.37 96.23) (width 0.2) (layer F.Cu) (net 14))
 (segment (start 209.689999 106.020001) (end 209.689999 97.549999) (width 0.2) (layer F.Cu) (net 14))
 (segment (start 208.89 106.82) (end 209.689999 106.020001) (width 0.2) (layer F.Cu) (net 14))
 (segment (start 255.479999 112.300001) (end 255.479999 95.917997) (width 0.2) (layer F.Cu) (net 1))
 (segment (start 253.34 114.44) (end 255.479999 112.300001) (width 0.2) (layer F.Cu) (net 1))
 (segment (start 255.479999 95.917997) (end 254.642001 95.079999) (width 0.2) (layer F.Cu) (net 1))
 (segment (start 254.642001 95.079999) (end 243.490001 95.079999) (width 0.2) (layer F.Cu) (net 1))
 (segment (start 243.490001 95.079999) (end 243.377999 95.079999) (width 0.2) (layer F.Cu) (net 1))
 (segment (start 226.702001 95.079999) (end 212.060001 95.079999) (width 0.2) (layer F.Cu) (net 1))
 (segment (start 227.539999 95.917997) (end 226.702001 95.079999) (width 0.2) (layer F.Cu) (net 1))
 (segment (start 228.377997 97.619999) (end 227.539999 96.782001) (width 0.2) (layer F.Cu) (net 1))
 (segment (start 229.840001 97.299999) (end 229.520001 97.619999) (width 0.2) (layer F.Cu) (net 1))
 (segment (start 227.539999 96.782001) (end 227.539999 95.917997) (width 0.2) (layer F.Cu) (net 1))
 (segment (start 229.840001 95.917997) (end 229.840001 97.299999) (width 0.2) (layer F.Cu) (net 1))
 (segment (start 230.677999 95.079999) (end 229.840001 95.917997) (width 0.2) (layer F.Cu) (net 1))
 (segment (start 212.060001 95.079999) (end 210.91 96.23) (width 0.2) (layer F.Cu) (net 1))
 (segment (start 229.520001 97.619999) (end 228.377997 97.619999) (width 0.2) (layer F.Cu) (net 1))
 (segment (start 243.490001 95.079999) (end 230.677999 95.079999) (width 0.2) (layer F.Cu) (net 1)))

